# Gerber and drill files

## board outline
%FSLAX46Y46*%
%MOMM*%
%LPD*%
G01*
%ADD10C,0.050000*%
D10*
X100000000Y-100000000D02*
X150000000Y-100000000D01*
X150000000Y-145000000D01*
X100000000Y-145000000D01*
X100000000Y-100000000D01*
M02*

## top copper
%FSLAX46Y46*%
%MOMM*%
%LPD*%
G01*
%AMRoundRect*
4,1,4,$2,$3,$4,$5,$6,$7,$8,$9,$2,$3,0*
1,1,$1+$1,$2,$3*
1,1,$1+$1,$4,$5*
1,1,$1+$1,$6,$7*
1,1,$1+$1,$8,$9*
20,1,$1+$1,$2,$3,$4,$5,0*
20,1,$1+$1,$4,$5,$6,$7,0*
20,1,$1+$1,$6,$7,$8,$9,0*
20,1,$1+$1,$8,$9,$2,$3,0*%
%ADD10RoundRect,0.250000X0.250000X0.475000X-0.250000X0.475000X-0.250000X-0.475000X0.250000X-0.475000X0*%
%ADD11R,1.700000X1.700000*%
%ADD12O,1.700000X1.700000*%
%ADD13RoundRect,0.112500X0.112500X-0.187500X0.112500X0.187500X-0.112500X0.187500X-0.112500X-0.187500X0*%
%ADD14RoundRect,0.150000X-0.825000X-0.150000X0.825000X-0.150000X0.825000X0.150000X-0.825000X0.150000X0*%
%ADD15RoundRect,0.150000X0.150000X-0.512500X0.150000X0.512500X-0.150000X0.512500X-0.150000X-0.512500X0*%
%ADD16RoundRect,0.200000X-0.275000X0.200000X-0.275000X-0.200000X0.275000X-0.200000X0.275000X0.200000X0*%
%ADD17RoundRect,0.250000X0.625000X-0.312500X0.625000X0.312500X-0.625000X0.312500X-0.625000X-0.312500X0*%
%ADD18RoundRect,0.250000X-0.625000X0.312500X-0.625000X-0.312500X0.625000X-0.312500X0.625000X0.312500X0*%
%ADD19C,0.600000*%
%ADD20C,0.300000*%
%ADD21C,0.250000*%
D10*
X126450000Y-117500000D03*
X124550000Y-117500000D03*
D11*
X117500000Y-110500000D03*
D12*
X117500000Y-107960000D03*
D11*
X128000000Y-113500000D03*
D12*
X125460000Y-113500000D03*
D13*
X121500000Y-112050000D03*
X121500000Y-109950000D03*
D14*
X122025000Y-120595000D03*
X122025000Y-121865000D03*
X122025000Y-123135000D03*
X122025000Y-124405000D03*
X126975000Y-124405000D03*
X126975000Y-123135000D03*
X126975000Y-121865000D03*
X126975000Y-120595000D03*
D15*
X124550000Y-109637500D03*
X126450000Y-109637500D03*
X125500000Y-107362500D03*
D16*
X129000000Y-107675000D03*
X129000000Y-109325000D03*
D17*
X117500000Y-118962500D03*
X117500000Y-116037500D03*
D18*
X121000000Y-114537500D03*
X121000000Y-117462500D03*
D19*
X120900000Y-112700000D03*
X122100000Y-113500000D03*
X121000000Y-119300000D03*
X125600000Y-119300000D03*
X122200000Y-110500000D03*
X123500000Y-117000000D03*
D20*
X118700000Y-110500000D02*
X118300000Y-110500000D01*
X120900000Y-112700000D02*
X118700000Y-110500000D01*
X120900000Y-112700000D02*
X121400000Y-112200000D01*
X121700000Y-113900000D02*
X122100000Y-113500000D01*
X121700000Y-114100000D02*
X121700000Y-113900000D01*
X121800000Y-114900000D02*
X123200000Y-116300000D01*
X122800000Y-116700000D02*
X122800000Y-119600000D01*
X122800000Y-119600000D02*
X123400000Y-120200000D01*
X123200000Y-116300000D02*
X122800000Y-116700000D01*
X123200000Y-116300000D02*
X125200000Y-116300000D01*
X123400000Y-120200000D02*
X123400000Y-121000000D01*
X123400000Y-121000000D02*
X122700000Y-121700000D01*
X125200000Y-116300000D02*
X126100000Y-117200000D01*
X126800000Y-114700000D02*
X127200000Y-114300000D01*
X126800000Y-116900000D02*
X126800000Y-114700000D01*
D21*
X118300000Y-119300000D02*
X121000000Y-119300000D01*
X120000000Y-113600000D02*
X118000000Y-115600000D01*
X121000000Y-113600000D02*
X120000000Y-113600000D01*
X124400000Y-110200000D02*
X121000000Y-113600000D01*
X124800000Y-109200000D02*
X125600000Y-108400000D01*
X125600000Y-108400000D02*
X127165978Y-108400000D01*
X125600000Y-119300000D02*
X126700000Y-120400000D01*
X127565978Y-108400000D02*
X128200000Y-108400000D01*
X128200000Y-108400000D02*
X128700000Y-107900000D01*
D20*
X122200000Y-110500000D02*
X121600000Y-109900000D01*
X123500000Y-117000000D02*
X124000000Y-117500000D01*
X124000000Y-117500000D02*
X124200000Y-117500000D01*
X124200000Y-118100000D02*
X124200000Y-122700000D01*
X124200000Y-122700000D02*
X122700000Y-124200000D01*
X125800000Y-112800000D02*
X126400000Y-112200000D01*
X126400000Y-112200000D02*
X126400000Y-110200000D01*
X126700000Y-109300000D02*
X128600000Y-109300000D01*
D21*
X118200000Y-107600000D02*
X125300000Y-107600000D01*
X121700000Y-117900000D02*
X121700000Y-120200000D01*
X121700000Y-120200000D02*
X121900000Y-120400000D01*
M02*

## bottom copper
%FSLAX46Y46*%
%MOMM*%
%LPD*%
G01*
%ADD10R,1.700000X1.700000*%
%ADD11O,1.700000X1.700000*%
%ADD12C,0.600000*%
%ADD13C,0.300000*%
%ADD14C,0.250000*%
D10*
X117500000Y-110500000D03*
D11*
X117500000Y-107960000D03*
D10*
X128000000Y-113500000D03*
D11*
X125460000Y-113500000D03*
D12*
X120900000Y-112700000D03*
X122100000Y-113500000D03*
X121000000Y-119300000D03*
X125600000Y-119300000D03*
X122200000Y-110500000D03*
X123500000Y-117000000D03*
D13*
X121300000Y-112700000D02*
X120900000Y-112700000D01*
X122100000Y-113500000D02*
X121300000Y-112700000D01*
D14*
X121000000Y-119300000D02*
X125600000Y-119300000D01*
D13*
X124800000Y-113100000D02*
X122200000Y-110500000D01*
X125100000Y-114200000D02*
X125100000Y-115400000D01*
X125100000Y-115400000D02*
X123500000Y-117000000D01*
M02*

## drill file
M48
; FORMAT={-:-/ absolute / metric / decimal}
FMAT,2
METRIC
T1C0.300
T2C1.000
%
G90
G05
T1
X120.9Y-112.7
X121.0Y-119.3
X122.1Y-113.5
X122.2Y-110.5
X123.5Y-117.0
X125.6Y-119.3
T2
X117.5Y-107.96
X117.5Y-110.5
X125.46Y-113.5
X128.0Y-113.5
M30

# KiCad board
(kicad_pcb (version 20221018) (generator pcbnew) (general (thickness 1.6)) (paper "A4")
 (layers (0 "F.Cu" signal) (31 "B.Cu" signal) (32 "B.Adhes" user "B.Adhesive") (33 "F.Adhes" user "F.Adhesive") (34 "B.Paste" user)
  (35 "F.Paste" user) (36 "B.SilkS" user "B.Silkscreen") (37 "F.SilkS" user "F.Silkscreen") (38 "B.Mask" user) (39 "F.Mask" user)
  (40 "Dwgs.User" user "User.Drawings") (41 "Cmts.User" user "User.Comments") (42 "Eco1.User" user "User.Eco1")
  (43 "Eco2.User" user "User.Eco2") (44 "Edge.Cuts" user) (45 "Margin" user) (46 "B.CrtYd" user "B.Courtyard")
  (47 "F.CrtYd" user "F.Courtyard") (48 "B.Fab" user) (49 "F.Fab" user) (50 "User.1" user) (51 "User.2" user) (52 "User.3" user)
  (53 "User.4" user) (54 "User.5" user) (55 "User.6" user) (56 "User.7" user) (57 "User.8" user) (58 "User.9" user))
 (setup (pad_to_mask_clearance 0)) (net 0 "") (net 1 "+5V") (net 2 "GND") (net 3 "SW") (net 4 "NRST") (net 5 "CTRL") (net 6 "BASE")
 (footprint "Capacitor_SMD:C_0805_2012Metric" (layer "F.Cu") (at 125.5 117.5 180)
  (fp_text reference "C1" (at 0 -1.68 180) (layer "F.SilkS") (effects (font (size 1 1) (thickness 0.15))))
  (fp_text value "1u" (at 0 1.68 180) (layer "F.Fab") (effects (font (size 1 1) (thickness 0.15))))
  (pad "1" smd roundrect (at -0.95 0 180) (size 1 1.45) (layers "F.Cu" "F.Paste" "F.Mask") (roundrect_rratio 0.25) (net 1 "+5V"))
  (pad "2" smd roundrect (at 0.95 0 180) (size 1 1.45) (layers "F.Cu" "F.Paste" "F.Mask") (roundrect_rratio 0.25) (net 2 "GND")))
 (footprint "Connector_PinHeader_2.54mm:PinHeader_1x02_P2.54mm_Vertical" (layer "F.Cu") (at 117.5 110.5 180)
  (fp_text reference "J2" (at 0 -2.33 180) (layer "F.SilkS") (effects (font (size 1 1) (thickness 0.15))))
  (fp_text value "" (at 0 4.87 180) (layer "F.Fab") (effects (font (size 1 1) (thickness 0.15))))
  (pad "1" thru_hole rect (at 0 0 180) (size 1.7 1.7) (drill 1) (layers "*.Cu" "*.Mask") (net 1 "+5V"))
  (pad "2" thru_hole oval (at 0 2.54 180) (size 1.7 1.7) (drill 1) (layers "*.Cu" "*.Mask") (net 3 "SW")))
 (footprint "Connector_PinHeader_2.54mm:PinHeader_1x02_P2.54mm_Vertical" (layer "F.Cu") (at 128 113.5 -90)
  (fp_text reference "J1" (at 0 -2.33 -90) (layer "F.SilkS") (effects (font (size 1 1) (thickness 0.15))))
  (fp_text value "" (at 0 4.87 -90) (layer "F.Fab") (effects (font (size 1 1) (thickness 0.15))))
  (pad "1" thru_hole rect (at 0 0 270) (size 1.7 1.7) (drill 1) (layers "*.Cu" "*.Mask") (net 1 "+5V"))
  (pad "2" thru_hole oval (at 0 2.54 270) (size 1.7 1.7) (drill 1) (layers "*.Cu" "*.Mask") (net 2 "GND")))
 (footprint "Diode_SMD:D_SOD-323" (layer "F.Cu") (at 121.5 111 90)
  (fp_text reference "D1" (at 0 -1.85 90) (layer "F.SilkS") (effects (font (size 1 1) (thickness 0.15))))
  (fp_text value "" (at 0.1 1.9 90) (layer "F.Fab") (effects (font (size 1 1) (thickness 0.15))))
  (pad "1" smd roundrect (at -1.05 0 90) (size 0.6 0.45) (layers "F.Cu" "F.Paste" "F.Mask") (roundrect_rratio 0.25) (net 1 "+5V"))
  (pad "2" smd roundrect (at 1.05 0 90) (size 0.6 0.45) (layers "F.Cu" "F.Paste" "F.Mask") (roundrect_rratio 0.25) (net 2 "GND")))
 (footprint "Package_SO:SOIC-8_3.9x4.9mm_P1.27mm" (layer "F.Cu") (at 124.5 122.5)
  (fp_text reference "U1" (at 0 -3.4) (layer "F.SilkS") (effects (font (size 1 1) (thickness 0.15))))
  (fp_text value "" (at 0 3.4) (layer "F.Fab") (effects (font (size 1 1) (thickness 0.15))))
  (pad "1" smd roundrect (at -2.475 -1.905) (size 1.95 0.6) (layers "F.Cu" "F.Paste" "F.Mask") (roundrect_rratio 0.25) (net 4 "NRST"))
  (pad "2" smd roundrect (at -2.475 -0.635) (size 1.95 0.6) (layers "F.Cu" "F.Paste" "F.Mask") (roundrect_rratio 0.25) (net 1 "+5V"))
  (pad "3" smd roundrect (at -2.475 0.635) (size 1.95 0.6) (layers "F.Cu" "F.Paste" "F.Mask") (roundrect_rratio 0.25))
  (pad "4" smd roundrect (at -2.475 1.905) (size 1.95 0.6) (layers "F.Cu" "F.Paste" "F.Mask") (roundrect_rratio 0.25) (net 2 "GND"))
  (pad "5" smd roundrect (at 2.475 1.905) (size 1.95 0.6) (layers "F.Cu" "F.Paste" "F.Mask") (roundrect_rratio 0.25))
  (pad "6" smd roundrect (at 2.475 0.635) (size 1.95 0.6) (layers "F.Cu" "F.Paste" "F.Mask") (roundrect_rratio 0.25))
  (pad "7" smd roundrect (at 2.475 -0.635) (size 1.95 0.6) (layers "F.Cu" "F.Paste" "F.Mask") (roundrect_rratio 0.25))
  (pad "8" smd roundrect (at 2.475 -1.905) (size 1.95 0.6) (layers "F.Cu" "F.Paste" "F.Mask") (roundrect_rratio 0.25) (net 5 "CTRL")))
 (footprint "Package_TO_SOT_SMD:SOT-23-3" (layer "F.Cu") (at 125.5 108.5 90)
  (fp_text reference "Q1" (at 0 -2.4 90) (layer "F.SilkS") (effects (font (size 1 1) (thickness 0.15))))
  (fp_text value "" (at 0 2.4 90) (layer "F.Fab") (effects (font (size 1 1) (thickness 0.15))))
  (pad "1" smd roundrect (at -1.1375 -0.95 90) (size 1.325 0.6) (layers "F.Cu" "F.Paste" "F.Mask") (roundrect_rratio 0.25) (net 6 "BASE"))
  (pad "2" smd roundrect (at -1.1375 0.95 90) (size 1.325 0.6) (layers "F.Cu" "F.Paste" "F.Mask") (roundrect_rratio 0.25) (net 2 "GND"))
  (pad "3" smd roundrect (at 1.1375 0 90) (size 1.325 0.6) (layers "F.Cu" "F.Paste" "F.Mask") (roundrect_rratio 0.25) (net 3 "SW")))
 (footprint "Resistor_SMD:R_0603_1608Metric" (layer "F.Cu") (at 129 108.5 -90)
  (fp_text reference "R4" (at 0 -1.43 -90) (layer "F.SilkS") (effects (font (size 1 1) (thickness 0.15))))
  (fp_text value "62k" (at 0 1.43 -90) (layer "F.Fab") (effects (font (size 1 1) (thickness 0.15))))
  (pad "1" smd roundrect (at -0.825 0 270) (size 0.8 0.95) (layers "F.Cu" "F.Paste" "F.Mask") (roundrect_rratio 0.25) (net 6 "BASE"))
  (pad "2" smd roundrect (at 0.825 0 270) (size 0.8 0.95) (layers "F.Cu" "F.Paste" "F.Mask") (roundrect_rratio 0.25) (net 2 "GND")))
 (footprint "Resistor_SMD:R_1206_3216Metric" (layer "F.Cu") (at 117.5 117.5 90)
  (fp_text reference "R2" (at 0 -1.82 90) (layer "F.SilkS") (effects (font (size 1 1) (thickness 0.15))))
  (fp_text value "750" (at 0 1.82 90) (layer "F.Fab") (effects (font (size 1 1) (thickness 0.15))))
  (pad "1" smd roundrect (at -1.4625 0 90) (size 1.125 1.75) (layers "F.Cu" "F.Paste" "F.Mask") (roundrect_rratio 0.222222) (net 5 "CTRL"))
  (pad "2" smd roundrect (at 1.4625 0 90) (size 1.125 1.75) (layers "F.Cu" "F.Paste" "F.Mask") (roundrect_rratio 0.222222) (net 6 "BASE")))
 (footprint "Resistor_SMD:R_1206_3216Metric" (layer "F.Cu") (at 121 116 -90)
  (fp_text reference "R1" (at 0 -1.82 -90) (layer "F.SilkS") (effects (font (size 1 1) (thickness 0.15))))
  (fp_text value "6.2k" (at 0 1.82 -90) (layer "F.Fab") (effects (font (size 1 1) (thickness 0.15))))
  (pad "1" smd roundrect (at -1.4625 0 270) (size 1.125 1.75) (layers "F.Cu" "F.Paste" "F.Mask") (roundrect_rratio 0.222222) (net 1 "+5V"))
  (pad "2" smd roundrect (at 1.4625 0 270) (size 1.125 1.75) (layers "F.Cu" "F.Paste" "F.Mask") (roundrect_rratio 0.222222) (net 4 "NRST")))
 (gr_rect (start 100 100) (end 150 145) (stroke (width 0.05) (type default)) (fill none) (layer "Edge.Cuts"))
 (segment (start 118.7 110.5) (end 118.3 110.5) (width 0.3) (layer "F.Cu") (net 1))
 (segment (start 120.9 112.7) (end 118.7 110.5) (width 0.3) (layer "F.Cu") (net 1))
 (segment (start 120.9 112.7) (end 121.4 112.2) (width 0.3) (layer "F.Cu") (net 1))
 (segment (start 121.7 113.9) (end 122.1 113.5) (width 0.3) (layer "F.Cu") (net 1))
 (segment (start 121.7 114.1) (end 121.7 113.9) (width 0.3) (layer "F.Cu") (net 1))
 (segment (start 121.8 114.9) (end 123.2 116.3) (width 0.3) (layer "F.Cu") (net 1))
 (segment (start 122.8 116.7) (end 122.8 119.6) (width 0.3) (layer "F.Cu") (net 1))
 (segment (start 122.8 119.6) (end 123.4 120.2) (width 0.3) (layer "F.Cu") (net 1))
 (segment (start 123.2 116.3) (end 122.8 116.7) (width 0.3) (layer "F.Cu") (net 1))
 (segment (start 123.2 116.3) (end 125.2 116.3) (width 0.3) (layer "F.Cu") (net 1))
 (segment (start 123.4 120.2) (end 123.4 121) (width 0.3) (layer "F.Cu") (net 1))
 (segment (start 123.4 121) (end 122.7 121.7) (width 0.3) (layer "F.Cu") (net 1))
 (segment (start 125.2 116.3) (end 126.1 117.2) (width 0.3) (layer "F.Cu") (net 1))
 (segment (start 126.8 114.7) (end 127.2 114.3) (width 0.3) (layer "F.Cu") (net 1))
 (segment (start 126.8 116.9) (end 126.8 114.7) (width 0.3) (layer "F.Cu") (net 1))
 (via (at 120.9 112.7) (size 0.6) (drill 0.3) (layers "F.Cu" "B.Cu") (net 1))
 (via (at 122.1 113.5) (size 0.6) (drill 0.3) (layers "F.Cu" "B.Cu") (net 1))
 (segment (start 118.3 119.3) (end 121 119.3) (width 0.25) (layer "F.Cu") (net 5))
 (segment (start 120 113.6) (end 118 115.6) (width 0.25) (layer "F.Cu") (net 6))
 (segment (start 121 113.6) (end 120 113.6) (width 0.25) (layer "F.Cu") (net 6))
 (segment (start 121.3 112.7) (end 120.9 112.7) (width 0.3) (layer "B.Cu") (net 1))
 (segment (start 122.1 113.5) (end 121.3 112.7) (width 0.3) (layer "B.Cu") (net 1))
 (segment (start 124.4 110.2) (end 121 113.6) (width 0.25) (layer "F.Cu") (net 6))
 (segment (start 124.8 109.2) (end 125.6 108.4) (width 0.25) (layer "F.Cu") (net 6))
 (segment (start 125.6 108.4) (end 127.165978 108.4) (width 0.25) (layer "F.Cu") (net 6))
 (segment (start 125.6 119.3) (end 126.7 120.4) (width 0.25) (layer "F.Cu") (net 5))
 (segment (start 127.565978 108.4) (end 128.2 108.4) (width 0.25) (layer "F.Cu") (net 6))
 (segment (start 128.2 108.4) (end 128.7 107.9) (width 0.25) (layer "F.Cu") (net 6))
 (via (at 121 119.3) (size 0.6) (drill 0.3) (layers "F.Cu" "B.Cu") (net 5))
 (via (at 125.6 119.3) (size 0.6) (drill 0.3) (layers "F.Cu" "B.Cu") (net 5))
 (segment (start 121 119.3) (end 125.6 119.3) (width 0.25) (layer "B.Cu") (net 5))
 (segment (start 122.2 110.5) (end 121.6 109.9) (width 0.3) (layer "F.Cu") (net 2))
 (segment (start 123.5 117) (end 124 117.5) (width 0.3) (layer "F.Cu") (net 2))
 (segment (start 124 117.5) (end 124.2 117.5) (width 0.3) (layer "F.Cu") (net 2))
 (segment (start 124.2 118.1) (end 124.2 122.7) (width 0.3) (layer "F.Cu") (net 2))
 (segment (start 124.2 122.7) (end 122.7 124.2) (width 0.3) (layer "F.Cu") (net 2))
 (segment (start 125.8 112.8) (end 126.4 112.2) (width 0.3) (layer "F.Cu") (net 2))
 (segment (start 126.4 112.2) (end 126.4 110.2) (width 0.3) (layer "F.Cu") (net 2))
 (segment (start 126.7 109.3) (end 128.6 109.3) (width 0.3) (layer "F.Cu") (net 2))
 (via (at 122.2 110.5) (size 0.6) (drill 0.3) (layers "F.Cu" "B.Cu") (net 2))
 (via (at 123.5 117) (size 0.6) (drill 0.3) (layers "F.Cu" "B.Cu") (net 2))
 (segment (start 118.2 107.6) (end 125.3 107.6) (width 0.25) (layer "F.Cu") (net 3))
 (segment (start 121.7 117.9) (end 121.7 120.2) (width 0.25) (layer "F.Cu") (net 4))
 (segment (start 121.7 120.2) (end 121.9 120.4) (width 0.25) (layer "F.Cu") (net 4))
 (segment (start 124.8 113.1) (end 122.2 110.5) (width 0.3) (layer "B.Cu") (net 2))
 (segment (start 125.1 114.2) (end 125.1 115.4) (width 0.3) (layer "B.Cu") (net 2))
 (segment (start 125.1 115.4) (end 123.5 117) (width 0.3) (layer "B.Cu") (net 2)))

